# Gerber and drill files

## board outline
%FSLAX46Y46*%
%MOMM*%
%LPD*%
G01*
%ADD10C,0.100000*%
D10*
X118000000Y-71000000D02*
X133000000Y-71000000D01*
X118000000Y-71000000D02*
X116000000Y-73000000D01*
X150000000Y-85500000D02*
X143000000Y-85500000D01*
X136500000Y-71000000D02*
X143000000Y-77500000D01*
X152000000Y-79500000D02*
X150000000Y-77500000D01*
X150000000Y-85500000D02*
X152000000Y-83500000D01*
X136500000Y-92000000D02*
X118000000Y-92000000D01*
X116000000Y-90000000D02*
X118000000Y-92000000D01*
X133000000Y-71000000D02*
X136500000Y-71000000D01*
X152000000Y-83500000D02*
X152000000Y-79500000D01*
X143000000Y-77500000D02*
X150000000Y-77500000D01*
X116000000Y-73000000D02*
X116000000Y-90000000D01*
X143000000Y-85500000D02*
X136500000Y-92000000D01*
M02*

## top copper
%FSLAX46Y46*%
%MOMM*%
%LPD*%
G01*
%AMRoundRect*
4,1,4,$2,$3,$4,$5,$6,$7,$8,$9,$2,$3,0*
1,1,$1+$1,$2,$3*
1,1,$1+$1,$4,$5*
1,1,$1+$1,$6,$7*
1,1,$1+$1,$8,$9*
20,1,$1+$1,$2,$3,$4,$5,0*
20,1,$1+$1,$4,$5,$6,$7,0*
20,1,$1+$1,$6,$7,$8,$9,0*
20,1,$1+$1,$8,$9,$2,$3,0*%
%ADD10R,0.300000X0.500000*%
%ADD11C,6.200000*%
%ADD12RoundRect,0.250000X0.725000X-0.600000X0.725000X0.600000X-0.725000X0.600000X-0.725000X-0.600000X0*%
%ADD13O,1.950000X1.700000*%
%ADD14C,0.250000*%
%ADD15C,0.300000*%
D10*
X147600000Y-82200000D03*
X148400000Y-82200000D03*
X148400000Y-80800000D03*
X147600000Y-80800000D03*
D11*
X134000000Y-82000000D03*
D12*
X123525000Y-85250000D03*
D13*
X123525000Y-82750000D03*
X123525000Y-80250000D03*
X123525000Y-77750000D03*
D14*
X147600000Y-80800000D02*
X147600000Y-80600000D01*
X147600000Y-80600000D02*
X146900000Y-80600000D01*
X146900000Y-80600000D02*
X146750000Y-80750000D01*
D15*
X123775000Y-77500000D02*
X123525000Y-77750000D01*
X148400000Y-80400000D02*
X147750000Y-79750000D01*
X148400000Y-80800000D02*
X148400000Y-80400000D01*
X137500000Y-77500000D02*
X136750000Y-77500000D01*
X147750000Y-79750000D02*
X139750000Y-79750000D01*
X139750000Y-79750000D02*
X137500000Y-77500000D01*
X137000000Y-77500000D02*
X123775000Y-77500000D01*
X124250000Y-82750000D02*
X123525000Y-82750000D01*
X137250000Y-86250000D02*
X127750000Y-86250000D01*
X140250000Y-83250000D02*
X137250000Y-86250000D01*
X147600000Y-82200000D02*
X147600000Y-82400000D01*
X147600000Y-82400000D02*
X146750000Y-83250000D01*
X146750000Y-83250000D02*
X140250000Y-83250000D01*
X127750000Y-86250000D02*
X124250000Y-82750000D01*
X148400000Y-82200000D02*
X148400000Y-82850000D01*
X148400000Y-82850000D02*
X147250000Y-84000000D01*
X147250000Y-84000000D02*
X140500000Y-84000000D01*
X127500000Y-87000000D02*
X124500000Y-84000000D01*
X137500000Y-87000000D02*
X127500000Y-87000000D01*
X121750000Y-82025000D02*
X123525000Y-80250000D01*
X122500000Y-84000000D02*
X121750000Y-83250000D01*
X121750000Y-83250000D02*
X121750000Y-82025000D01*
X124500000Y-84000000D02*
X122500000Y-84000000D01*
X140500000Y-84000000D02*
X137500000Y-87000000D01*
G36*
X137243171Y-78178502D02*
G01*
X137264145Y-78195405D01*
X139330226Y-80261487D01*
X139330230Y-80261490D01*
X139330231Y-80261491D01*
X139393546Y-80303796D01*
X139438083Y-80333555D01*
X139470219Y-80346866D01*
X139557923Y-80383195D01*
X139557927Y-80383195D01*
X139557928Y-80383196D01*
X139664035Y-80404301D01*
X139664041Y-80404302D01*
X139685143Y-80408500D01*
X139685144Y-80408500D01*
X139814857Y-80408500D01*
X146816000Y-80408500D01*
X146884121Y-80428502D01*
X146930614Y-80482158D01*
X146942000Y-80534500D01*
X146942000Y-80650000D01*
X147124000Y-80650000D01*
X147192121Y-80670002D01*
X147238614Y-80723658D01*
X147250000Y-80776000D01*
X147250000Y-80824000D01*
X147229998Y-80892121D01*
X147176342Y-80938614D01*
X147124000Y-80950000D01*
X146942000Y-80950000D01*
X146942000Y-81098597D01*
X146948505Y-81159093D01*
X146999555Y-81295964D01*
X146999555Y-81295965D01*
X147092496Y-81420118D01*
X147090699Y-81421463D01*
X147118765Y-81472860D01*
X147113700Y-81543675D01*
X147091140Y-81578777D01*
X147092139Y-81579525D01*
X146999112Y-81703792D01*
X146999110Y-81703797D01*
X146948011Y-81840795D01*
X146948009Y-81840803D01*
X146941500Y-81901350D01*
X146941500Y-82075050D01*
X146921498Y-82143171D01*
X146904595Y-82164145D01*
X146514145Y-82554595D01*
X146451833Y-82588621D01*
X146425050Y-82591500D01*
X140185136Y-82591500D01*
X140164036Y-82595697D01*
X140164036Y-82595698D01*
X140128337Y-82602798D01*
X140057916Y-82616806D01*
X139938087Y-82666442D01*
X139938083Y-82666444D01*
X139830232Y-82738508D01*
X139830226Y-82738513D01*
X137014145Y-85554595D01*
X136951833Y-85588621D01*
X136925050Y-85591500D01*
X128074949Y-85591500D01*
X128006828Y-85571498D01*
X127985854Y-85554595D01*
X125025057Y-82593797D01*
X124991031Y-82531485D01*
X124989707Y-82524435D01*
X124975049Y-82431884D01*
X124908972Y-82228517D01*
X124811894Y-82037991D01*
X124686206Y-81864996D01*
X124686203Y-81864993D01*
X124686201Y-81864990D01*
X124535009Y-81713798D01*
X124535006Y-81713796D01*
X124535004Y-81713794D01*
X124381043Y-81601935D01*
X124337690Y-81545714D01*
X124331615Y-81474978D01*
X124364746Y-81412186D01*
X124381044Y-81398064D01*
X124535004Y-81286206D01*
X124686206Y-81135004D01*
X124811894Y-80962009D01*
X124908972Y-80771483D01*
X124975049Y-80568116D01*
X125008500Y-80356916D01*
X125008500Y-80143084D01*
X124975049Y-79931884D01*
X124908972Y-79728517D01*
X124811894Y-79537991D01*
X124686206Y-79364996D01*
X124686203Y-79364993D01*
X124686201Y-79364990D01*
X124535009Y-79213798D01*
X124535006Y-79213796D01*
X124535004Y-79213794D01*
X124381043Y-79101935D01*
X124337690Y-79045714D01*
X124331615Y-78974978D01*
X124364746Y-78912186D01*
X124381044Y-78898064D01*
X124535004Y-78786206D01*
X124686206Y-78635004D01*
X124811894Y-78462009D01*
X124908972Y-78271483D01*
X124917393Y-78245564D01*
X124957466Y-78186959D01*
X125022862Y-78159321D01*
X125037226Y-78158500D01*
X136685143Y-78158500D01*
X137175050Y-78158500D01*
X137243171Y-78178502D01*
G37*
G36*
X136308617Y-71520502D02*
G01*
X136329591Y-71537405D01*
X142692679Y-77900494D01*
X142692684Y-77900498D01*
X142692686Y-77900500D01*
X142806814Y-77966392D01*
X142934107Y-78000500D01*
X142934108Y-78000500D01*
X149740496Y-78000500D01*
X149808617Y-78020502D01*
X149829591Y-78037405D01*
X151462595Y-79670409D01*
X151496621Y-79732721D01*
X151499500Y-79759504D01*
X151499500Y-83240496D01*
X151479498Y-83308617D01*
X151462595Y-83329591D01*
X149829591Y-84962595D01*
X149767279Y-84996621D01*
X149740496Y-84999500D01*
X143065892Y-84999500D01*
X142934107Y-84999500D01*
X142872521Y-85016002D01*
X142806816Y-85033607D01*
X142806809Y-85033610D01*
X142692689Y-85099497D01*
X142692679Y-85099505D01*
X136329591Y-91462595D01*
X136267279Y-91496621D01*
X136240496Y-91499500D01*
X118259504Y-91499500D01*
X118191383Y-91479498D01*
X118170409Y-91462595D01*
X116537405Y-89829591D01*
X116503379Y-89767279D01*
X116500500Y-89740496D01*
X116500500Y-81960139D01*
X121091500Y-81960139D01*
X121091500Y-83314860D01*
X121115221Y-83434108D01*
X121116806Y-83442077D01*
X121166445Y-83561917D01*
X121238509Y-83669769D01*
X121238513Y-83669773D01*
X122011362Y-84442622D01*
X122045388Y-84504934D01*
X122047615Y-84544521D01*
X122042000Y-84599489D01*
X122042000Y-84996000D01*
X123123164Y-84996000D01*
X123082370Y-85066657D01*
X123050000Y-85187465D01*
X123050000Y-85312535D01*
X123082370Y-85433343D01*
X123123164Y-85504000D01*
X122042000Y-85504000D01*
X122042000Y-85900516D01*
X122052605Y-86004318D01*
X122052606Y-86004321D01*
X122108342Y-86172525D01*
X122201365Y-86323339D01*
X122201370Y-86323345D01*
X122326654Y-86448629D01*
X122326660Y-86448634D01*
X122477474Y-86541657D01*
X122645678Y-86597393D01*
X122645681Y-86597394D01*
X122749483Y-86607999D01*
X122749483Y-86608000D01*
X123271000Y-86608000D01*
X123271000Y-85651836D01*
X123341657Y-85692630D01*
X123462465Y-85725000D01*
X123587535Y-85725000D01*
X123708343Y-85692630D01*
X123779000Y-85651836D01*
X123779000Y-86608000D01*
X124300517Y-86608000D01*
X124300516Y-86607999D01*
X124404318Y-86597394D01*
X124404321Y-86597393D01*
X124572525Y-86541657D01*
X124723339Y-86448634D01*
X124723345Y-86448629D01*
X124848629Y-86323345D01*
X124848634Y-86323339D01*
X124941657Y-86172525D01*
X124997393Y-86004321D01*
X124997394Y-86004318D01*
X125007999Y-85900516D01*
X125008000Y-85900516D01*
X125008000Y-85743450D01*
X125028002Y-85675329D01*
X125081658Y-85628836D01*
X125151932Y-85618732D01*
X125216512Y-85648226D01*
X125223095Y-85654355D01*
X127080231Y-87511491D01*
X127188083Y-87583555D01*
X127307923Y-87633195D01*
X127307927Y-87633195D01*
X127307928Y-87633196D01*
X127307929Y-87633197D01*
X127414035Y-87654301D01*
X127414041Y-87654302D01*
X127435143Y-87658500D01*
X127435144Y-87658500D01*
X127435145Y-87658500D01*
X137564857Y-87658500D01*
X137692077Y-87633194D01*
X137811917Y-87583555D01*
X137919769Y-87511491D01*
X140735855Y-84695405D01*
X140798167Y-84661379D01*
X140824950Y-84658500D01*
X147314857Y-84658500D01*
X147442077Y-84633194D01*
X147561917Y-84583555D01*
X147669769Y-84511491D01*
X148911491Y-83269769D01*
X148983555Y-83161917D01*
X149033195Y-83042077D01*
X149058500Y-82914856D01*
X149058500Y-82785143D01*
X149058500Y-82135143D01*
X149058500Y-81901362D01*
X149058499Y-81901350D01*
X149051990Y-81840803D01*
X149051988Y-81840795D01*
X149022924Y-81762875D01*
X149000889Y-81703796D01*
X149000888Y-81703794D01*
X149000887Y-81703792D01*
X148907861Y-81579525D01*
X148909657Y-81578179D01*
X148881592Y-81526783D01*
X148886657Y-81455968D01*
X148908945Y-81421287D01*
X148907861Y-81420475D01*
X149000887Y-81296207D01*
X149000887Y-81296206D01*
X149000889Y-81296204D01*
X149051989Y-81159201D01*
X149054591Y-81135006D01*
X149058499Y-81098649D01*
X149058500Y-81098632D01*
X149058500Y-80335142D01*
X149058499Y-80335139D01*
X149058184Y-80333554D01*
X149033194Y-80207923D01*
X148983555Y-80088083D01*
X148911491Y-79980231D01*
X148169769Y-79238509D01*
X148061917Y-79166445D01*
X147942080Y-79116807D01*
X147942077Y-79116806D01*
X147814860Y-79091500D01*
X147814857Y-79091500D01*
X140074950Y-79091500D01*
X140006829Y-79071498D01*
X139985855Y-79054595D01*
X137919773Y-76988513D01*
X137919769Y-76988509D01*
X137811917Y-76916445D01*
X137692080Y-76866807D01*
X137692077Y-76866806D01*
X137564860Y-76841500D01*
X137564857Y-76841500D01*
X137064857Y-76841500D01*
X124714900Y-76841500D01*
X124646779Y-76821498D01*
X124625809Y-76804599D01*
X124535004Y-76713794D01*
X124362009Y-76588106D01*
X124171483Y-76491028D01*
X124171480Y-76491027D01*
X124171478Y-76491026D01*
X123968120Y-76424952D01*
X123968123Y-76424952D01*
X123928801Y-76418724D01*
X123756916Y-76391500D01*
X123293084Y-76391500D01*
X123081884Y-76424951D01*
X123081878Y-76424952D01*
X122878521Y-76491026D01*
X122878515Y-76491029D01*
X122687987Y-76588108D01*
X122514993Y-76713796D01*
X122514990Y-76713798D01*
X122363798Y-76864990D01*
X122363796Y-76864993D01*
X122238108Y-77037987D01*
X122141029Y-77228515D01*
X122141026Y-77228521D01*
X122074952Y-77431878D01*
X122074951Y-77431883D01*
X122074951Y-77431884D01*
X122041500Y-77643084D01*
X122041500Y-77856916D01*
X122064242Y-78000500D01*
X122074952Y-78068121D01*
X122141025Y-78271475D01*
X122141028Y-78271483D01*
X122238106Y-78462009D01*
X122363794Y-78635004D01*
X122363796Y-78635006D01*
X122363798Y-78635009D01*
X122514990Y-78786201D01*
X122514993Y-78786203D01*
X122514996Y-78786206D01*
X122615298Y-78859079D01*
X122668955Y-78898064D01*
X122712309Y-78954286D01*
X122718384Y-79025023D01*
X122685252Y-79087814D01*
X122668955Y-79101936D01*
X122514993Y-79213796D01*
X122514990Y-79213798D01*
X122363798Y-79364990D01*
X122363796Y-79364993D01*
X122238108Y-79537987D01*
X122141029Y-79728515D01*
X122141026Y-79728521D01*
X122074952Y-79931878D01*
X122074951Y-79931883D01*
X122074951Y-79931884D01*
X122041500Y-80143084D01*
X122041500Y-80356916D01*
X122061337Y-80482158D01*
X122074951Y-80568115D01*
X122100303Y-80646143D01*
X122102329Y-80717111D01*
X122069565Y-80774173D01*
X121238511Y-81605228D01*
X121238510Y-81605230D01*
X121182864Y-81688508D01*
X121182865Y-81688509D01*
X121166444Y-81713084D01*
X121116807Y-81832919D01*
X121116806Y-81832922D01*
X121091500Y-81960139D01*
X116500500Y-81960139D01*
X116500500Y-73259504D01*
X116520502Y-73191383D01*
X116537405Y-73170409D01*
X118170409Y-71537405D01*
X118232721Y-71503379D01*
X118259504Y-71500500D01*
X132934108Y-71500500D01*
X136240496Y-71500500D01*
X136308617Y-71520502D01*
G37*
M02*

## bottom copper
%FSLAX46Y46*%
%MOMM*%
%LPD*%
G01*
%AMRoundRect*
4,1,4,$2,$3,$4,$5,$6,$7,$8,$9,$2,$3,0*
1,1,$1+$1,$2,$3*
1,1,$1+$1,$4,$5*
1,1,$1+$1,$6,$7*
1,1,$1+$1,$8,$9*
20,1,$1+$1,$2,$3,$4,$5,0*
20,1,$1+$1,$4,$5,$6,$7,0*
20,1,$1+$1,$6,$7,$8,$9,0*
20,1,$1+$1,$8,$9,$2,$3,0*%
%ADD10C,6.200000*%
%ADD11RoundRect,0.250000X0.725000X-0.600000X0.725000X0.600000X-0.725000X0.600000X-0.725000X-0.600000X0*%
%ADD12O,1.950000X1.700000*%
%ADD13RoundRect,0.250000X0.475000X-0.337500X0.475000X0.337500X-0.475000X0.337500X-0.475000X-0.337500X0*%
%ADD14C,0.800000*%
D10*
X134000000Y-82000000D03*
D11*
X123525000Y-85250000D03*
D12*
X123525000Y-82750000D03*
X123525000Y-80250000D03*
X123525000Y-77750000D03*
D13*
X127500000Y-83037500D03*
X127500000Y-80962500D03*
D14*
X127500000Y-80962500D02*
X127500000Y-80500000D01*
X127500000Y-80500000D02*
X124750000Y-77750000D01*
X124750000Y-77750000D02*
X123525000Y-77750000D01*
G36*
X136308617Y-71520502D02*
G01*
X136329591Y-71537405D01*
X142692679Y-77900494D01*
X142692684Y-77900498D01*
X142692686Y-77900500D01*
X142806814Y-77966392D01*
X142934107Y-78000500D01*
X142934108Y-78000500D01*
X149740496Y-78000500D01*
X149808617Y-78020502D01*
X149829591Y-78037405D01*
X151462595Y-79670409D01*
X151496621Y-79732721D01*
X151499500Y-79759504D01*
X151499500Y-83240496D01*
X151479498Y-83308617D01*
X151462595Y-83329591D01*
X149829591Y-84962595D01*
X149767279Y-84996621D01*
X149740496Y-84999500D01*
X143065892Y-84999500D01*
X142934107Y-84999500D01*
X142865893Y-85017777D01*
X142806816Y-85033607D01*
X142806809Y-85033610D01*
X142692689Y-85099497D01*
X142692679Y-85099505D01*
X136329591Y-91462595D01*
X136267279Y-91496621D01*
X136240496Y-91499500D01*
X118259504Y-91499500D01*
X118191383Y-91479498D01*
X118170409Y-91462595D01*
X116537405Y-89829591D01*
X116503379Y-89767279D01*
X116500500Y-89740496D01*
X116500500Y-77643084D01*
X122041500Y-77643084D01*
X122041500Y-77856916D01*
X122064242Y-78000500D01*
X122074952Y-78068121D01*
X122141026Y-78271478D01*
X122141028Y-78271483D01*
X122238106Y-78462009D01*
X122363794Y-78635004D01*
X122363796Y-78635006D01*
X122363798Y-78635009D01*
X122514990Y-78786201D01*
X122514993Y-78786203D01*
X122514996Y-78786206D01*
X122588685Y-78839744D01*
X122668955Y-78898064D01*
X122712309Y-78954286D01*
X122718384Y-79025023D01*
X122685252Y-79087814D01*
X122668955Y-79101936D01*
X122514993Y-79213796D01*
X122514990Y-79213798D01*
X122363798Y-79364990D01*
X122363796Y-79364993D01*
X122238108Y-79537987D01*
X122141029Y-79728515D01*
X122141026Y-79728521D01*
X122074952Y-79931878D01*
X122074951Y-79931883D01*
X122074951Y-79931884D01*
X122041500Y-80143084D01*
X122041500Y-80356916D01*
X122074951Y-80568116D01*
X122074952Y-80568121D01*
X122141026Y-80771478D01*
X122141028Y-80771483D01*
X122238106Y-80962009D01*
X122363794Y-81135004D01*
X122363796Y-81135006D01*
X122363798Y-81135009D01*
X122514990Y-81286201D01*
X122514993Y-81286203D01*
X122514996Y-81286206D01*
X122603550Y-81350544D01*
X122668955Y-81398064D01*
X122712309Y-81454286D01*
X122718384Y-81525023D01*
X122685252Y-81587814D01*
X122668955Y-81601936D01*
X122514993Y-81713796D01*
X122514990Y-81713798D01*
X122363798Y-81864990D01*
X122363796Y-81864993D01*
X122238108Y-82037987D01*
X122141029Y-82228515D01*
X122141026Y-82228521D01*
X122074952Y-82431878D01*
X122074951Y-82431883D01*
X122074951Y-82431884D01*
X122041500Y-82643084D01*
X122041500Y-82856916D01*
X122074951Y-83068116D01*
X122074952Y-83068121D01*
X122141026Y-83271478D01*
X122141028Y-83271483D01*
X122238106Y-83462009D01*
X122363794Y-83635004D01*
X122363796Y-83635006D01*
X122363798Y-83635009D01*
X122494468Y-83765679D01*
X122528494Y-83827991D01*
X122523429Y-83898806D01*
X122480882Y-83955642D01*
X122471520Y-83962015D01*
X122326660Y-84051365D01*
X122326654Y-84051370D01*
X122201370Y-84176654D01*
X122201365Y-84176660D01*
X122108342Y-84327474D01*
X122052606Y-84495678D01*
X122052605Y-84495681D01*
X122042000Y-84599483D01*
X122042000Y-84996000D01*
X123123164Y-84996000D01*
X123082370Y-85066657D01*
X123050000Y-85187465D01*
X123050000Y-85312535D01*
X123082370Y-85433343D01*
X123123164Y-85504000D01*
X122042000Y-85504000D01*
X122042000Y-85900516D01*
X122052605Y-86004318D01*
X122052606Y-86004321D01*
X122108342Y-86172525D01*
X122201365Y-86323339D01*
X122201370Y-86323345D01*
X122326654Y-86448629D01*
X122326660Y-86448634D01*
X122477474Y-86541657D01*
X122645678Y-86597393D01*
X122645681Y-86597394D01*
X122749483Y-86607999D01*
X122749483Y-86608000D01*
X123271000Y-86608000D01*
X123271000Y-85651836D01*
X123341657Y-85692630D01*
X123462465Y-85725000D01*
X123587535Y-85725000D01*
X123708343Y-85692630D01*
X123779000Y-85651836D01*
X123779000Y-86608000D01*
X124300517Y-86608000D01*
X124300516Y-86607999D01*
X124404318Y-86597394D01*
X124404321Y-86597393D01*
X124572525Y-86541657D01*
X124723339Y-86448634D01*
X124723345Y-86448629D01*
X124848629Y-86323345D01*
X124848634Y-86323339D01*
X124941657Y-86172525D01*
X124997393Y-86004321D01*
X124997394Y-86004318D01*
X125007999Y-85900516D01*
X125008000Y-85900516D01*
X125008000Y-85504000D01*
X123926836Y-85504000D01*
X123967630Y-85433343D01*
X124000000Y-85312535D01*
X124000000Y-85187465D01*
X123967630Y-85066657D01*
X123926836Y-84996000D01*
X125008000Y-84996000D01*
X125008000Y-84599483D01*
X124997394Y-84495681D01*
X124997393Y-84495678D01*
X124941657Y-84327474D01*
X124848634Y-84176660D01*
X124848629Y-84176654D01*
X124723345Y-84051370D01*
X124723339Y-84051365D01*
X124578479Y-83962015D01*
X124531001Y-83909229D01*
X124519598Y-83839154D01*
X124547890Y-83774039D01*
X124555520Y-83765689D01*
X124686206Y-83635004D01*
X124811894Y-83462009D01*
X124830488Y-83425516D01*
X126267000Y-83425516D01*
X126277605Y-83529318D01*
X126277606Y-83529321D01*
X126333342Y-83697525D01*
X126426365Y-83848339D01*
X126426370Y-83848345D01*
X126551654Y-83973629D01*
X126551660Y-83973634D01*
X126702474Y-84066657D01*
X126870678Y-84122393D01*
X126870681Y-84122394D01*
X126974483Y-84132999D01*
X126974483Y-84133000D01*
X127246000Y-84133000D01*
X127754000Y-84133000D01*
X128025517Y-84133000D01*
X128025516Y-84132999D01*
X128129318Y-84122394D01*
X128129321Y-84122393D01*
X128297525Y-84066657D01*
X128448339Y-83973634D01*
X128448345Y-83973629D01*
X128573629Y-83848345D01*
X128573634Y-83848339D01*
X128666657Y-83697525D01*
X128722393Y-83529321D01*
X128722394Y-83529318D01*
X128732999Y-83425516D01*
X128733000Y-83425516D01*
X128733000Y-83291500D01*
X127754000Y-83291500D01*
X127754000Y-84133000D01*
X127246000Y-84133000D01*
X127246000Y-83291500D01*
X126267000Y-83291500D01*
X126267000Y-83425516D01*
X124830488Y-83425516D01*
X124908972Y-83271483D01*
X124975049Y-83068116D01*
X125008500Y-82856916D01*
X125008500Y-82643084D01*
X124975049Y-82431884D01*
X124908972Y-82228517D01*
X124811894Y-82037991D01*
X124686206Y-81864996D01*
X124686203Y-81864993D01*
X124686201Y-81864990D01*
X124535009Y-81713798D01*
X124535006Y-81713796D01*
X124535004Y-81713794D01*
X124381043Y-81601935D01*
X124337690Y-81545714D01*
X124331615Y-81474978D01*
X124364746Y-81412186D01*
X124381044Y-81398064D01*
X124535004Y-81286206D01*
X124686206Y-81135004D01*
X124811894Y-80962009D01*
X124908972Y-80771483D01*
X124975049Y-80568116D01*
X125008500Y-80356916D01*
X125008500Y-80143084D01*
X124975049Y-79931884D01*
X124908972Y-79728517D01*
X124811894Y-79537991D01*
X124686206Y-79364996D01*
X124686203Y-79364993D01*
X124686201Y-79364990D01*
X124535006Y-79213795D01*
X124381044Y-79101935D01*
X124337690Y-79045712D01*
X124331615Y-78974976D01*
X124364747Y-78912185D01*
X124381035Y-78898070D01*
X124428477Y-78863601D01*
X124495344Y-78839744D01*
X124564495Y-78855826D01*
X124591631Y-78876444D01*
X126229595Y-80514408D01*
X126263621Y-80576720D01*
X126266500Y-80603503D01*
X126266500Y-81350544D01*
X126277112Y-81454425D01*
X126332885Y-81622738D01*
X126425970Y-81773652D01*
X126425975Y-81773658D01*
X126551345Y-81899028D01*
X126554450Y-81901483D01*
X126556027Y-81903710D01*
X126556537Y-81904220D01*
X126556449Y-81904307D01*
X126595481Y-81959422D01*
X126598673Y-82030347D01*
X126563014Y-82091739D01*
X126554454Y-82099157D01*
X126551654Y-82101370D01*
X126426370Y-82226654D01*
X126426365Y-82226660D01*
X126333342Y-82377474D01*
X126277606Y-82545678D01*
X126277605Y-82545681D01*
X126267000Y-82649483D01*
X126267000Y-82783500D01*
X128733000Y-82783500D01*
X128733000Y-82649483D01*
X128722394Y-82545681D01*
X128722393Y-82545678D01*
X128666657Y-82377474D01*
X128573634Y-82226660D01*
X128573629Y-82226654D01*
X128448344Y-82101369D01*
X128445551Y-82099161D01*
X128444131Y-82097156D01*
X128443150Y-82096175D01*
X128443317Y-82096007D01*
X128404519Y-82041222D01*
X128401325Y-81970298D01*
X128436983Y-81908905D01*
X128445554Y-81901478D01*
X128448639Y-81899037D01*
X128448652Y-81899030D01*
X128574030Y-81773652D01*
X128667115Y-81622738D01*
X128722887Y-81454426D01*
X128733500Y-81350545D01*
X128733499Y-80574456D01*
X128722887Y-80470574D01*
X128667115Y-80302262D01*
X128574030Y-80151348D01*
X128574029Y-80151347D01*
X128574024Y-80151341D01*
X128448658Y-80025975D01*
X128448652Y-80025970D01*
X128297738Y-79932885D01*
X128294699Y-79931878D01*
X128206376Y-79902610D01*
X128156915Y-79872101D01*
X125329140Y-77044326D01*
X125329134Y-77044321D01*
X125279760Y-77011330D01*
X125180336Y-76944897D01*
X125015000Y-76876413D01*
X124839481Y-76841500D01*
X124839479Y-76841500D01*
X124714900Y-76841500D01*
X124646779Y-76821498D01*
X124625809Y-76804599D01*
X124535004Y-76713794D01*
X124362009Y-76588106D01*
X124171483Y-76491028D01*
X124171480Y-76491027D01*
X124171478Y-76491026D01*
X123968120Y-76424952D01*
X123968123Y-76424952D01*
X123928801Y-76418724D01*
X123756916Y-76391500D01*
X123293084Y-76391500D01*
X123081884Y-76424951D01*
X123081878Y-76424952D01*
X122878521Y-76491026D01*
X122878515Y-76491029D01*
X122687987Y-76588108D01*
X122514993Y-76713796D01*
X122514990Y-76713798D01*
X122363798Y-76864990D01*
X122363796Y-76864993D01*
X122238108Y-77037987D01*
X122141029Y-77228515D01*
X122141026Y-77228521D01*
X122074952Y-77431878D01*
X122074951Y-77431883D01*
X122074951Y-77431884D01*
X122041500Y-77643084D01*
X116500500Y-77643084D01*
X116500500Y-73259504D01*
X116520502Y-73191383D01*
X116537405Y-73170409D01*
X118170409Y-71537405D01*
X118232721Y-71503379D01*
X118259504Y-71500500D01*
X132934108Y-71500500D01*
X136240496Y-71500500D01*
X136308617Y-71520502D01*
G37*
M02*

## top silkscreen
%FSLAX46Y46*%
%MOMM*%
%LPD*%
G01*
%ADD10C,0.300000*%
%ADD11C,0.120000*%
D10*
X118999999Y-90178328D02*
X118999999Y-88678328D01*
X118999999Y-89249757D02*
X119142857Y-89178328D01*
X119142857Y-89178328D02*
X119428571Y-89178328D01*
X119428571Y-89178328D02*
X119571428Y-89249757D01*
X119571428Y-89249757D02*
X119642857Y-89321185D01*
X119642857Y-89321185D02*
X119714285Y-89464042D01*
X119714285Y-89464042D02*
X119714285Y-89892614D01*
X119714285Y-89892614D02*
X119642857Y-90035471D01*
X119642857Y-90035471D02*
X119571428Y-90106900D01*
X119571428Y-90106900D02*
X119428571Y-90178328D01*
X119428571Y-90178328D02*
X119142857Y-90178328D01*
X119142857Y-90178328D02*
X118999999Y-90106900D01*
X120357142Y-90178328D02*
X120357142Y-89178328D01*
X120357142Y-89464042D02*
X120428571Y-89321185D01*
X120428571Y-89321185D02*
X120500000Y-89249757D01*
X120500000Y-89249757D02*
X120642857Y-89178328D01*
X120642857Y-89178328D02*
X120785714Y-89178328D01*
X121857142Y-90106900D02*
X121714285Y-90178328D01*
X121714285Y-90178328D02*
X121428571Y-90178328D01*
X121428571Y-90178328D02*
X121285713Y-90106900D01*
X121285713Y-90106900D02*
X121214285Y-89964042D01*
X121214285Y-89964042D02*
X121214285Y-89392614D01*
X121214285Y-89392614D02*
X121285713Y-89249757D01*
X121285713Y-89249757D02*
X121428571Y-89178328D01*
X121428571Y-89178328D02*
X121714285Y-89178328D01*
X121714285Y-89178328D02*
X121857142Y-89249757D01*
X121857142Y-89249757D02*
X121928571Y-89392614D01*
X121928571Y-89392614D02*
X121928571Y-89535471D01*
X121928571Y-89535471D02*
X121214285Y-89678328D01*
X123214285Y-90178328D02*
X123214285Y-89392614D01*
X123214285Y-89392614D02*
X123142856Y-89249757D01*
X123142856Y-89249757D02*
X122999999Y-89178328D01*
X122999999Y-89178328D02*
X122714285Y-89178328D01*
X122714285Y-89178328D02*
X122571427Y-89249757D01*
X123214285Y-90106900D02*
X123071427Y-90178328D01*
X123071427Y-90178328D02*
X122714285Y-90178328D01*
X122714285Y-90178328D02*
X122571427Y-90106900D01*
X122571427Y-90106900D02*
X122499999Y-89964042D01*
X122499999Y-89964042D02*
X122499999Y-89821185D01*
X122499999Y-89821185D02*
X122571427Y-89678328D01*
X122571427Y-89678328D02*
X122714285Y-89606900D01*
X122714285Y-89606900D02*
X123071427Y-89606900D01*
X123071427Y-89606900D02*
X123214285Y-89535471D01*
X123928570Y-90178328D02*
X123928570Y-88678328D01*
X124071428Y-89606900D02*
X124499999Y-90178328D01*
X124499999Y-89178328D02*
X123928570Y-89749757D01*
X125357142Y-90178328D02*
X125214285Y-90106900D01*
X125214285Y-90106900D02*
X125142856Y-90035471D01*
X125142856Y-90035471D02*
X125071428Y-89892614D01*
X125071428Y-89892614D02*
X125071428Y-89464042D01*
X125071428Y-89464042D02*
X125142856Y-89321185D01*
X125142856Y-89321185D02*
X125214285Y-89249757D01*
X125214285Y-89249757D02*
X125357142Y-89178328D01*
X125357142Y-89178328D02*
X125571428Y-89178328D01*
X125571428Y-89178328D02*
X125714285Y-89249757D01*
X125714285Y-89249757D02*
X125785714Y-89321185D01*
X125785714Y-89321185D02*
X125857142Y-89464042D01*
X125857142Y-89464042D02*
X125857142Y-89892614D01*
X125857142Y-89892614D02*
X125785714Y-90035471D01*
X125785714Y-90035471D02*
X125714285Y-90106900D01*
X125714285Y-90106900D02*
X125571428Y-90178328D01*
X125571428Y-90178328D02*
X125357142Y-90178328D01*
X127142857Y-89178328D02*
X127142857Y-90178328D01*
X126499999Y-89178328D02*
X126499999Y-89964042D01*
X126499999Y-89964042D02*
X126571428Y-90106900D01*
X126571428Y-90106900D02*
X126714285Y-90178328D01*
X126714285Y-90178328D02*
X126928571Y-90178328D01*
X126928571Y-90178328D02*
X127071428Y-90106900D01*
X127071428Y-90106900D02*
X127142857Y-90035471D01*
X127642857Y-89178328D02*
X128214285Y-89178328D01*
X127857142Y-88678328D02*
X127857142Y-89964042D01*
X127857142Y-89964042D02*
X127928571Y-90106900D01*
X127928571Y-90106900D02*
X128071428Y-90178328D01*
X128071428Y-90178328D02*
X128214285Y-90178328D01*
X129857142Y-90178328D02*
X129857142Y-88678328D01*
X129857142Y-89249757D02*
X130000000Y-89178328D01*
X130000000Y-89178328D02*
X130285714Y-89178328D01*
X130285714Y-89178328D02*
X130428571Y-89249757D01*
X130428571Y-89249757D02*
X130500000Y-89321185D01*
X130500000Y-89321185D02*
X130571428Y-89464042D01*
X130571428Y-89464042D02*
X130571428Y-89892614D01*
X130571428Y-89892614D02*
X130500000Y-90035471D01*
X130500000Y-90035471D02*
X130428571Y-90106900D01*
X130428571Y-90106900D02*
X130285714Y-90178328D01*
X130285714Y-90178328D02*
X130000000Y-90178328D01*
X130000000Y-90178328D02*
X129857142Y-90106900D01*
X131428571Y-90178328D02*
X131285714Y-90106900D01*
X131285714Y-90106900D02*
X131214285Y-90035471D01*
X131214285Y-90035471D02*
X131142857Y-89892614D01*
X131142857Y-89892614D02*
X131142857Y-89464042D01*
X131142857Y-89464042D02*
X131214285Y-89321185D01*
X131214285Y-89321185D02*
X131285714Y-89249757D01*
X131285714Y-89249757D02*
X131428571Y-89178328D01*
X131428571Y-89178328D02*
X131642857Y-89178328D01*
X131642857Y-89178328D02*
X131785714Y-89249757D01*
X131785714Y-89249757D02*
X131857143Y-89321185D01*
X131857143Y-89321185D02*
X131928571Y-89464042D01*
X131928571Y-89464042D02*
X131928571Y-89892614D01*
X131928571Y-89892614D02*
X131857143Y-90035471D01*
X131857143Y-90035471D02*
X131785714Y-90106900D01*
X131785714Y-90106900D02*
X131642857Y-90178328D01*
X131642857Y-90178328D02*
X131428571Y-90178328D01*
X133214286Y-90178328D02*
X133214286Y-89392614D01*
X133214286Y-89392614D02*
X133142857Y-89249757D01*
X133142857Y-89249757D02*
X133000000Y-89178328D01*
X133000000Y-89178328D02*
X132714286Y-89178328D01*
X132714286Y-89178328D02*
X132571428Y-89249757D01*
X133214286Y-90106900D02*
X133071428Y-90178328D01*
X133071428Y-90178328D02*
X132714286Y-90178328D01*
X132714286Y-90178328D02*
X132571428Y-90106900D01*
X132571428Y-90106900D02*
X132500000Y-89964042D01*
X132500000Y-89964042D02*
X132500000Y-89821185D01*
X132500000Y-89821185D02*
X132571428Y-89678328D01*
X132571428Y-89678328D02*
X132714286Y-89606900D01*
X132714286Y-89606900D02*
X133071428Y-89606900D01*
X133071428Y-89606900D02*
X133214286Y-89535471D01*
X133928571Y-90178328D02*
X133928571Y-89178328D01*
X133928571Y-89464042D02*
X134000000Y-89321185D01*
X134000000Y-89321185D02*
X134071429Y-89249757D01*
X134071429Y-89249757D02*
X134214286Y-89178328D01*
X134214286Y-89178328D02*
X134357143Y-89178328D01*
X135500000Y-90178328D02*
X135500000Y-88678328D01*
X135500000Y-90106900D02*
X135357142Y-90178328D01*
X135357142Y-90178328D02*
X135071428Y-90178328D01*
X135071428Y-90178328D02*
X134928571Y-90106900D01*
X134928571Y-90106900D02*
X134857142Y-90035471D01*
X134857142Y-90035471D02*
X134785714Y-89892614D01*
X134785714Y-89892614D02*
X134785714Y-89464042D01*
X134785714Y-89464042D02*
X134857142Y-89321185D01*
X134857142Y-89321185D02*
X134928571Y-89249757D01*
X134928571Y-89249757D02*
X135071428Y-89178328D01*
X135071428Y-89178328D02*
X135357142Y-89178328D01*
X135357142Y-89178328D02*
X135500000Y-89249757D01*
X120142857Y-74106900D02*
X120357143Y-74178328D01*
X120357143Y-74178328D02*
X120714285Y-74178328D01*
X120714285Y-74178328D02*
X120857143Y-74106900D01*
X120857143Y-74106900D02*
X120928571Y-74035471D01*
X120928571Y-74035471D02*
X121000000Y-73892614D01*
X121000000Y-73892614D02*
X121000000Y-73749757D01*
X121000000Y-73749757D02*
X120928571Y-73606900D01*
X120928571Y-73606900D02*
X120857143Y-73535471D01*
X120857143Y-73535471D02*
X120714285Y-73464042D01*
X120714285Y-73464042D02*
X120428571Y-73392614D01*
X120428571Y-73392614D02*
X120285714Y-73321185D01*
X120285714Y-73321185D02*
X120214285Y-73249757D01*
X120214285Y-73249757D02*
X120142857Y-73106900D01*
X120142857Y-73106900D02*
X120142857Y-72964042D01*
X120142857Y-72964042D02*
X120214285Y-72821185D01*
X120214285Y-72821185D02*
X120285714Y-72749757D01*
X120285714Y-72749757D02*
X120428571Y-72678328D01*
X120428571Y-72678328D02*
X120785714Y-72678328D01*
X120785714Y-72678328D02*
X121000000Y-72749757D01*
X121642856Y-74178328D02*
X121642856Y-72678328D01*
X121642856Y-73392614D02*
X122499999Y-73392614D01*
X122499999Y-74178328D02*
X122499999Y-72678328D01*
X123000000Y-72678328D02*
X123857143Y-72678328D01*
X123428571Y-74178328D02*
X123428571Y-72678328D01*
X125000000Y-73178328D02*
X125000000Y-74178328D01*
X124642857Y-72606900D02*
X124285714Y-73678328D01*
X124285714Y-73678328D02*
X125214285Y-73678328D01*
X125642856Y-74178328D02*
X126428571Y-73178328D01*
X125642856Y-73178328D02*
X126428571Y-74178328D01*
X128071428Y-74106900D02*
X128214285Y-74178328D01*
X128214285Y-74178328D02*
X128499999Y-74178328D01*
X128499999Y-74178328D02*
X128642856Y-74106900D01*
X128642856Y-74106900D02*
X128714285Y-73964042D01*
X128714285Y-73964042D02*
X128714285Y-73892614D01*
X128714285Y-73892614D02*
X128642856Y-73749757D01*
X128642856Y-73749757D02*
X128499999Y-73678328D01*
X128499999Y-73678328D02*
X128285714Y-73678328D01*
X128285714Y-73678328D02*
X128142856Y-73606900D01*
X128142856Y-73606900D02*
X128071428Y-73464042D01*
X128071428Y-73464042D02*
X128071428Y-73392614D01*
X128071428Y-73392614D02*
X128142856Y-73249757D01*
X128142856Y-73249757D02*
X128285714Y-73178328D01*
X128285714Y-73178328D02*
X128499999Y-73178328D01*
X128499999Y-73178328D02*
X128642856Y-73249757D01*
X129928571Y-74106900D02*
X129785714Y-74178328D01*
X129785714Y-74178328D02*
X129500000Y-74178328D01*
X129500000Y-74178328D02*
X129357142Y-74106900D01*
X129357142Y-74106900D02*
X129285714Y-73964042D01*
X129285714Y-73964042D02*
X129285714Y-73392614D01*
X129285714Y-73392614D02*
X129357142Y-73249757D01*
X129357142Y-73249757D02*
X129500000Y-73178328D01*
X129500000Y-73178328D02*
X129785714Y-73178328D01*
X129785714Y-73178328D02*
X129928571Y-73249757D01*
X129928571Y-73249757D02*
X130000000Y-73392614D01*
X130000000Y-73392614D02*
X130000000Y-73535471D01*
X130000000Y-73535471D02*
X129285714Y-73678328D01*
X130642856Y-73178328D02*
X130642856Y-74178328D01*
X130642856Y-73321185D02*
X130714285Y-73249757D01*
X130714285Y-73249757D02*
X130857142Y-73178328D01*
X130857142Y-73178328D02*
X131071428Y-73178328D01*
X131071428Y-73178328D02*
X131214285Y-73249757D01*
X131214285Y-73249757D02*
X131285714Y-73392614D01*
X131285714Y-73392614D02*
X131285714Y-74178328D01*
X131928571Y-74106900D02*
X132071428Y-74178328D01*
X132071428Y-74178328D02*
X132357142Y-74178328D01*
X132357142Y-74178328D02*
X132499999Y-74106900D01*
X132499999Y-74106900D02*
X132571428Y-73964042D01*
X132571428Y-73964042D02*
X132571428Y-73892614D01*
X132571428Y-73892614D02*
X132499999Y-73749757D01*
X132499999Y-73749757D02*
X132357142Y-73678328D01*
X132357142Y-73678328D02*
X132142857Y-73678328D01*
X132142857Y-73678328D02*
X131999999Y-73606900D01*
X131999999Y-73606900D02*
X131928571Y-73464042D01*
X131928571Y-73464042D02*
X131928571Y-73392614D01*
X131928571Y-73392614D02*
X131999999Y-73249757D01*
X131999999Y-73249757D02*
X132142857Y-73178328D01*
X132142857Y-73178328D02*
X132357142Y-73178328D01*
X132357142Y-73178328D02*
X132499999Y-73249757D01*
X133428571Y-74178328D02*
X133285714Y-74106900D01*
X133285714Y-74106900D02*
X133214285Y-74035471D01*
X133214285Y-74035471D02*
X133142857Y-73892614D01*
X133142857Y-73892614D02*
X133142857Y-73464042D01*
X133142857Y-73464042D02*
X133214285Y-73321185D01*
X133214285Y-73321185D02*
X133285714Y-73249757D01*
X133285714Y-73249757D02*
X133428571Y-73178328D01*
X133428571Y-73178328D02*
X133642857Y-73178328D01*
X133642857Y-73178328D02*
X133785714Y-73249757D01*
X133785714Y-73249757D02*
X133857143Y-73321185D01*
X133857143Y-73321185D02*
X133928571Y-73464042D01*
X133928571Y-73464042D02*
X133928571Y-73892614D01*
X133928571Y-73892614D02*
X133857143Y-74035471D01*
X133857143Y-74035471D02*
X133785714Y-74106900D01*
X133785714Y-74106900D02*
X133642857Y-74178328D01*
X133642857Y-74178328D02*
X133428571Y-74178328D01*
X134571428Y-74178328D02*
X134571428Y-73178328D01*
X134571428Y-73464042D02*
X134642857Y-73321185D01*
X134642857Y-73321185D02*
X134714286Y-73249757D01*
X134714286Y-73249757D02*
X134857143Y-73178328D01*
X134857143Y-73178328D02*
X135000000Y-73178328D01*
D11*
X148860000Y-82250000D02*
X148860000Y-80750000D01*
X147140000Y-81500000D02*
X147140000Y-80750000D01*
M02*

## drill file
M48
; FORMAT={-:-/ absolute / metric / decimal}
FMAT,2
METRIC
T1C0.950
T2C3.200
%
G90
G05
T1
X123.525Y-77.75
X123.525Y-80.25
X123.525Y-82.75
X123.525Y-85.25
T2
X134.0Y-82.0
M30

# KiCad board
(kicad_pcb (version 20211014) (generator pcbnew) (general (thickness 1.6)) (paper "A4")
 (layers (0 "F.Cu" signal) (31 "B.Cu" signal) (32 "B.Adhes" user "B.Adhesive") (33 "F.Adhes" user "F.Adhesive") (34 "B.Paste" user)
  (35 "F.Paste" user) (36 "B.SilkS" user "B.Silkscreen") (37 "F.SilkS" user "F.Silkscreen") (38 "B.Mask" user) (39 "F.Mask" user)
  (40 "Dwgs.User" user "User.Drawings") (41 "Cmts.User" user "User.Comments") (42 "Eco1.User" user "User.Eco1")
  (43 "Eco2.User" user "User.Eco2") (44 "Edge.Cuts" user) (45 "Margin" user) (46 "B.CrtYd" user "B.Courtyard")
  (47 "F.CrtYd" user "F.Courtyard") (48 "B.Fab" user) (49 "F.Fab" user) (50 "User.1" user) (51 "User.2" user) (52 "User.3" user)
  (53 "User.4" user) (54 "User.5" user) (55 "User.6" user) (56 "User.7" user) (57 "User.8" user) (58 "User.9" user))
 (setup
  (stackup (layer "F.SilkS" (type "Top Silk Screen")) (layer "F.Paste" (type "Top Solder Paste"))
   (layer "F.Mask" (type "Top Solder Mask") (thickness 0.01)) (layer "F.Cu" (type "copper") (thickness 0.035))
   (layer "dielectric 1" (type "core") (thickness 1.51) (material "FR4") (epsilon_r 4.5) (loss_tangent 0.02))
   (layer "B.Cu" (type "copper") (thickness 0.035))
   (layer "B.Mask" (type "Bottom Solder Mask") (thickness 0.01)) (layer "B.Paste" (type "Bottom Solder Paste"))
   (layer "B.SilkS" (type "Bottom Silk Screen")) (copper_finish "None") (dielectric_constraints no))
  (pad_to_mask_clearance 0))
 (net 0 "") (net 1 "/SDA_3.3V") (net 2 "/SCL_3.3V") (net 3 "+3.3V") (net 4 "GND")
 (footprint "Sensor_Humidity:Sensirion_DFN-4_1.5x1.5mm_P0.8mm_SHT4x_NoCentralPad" (layer "F.Cu") (at 148 81.5 90)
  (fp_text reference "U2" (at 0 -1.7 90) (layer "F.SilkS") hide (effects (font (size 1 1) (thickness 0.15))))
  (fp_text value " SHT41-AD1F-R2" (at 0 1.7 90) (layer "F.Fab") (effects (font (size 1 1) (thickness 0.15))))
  (fp_line (start -0.75 0.86) (end 0.75 0.86) (layer "F.SilkS") (width 0.12))
  (fp_line (start 0 -0.86) (end 0.75 -0.86) (layer "F.SilkS") (width 0.12))
  (pad "1" smd rect (at -0.7 -0.4 90) (size 0.5 0.3) (layers "F.Cu" "F.Paste" "F.Mask") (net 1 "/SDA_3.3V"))
  (pad "2" smd rect (at -0.7 0.4 90) (size 0.5 0.3) (layers "F.Cu" "F.Paste" "F.Mask") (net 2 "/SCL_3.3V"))
  (pad "3" smd rect (at 0.7 0.4 90) (size 0.5 0.3) (layers "F.Cu" "F.Paste" "F.Mask") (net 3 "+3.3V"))
  (pad "4" smd rect (at 0.7 -0.4 90) (size 0.5 0.3) (layers "F.Cu" "F.Paste" "F.Mask") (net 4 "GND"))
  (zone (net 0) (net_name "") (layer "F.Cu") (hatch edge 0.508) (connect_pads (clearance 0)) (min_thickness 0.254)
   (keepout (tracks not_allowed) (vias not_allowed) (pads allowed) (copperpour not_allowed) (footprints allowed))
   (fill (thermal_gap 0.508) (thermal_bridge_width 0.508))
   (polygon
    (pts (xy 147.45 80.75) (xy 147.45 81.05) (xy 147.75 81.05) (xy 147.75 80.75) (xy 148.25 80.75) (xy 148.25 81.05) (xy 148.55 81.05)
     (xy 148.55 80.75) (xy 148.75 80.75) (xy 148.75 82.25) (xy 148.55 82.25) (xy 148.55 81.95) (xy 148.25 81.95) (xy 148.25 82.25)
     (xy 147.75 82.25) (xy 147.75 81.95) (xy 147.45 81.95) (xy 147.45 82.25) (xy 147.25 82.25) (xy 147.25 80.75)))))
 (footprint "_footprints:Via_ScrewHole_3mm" (layer "F.Cu") (at 134 82)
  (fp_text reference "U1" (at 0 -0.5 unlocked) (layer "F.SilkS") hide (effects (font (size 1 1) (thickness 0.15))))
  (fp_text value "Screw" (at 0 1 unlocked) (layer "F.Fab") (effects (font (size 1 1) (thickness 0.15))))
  (pad "1" thru_hole circle (at 0 0) (size 6.2 6.2) (drill 3.2) (layers *.Cu *.Mask) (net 4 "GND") (zone_connect 2)))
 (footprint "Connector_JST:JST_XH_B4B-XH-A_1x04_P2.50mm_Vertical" (layer "B.Cu") (at 123.525 85.25 90)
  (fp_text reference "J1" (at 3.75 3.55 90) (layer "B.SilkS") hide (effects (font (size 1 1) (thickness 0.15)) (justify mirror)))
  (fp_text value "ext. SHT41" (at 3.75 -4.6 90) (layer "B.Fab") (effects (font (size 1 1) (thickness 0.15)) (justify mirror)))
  (pad "1" thru_hole roundrect (at 0 0 90) (size 1.7 1.95) (drill 0.95) (layers *.Cu *.Mask) (roundrect_rratio 0.1470588235) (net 4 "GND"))
  (pad "2" thru_hole oval (at 2.5 0 90) (size 1.7 1.95) (drill 0.95) (layers *.Cu *.Mask) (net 1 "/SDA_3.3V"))
  (pad "3" thru_hole oval (at 5 0 90) (size 1.7 1.95) (drill 0.95) (layers *.Cu *.Mask) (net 2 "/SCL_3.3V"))
  (pad "4" thru_hole oval (at 7.5 0 90) (size 1.7 1.95) (drill 0.95) (layers *.Cu *.Mask) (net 3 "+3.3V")))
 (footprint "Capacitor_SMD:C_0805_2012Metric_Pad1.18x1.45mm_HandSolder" (layer "B.Cu") (at 127.5 82 90)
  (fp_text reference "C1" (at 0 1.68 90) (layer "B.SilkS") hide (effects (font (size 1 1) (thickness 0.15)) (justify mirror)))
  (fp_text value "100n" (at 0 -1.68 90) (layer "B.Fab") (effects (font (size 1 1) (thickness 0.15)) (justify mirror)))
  (pad "1" smd roundrect (at -1.0375 0 90) (size 1.175 1.45) (layers "B.Cu" "B.Paste" "B.Mask") (roundrect_rratio 0.2127659574)
   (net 4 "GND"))
  (pad "2" smd roundrect (at 1.0375 0 90) (size 1.175 1.45) (layers "B.Cu" "B.Paste" "B.Mask") (roundrect_rratio 0.2127659574)
   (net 3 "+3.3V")))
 (gr_line (start 118 71) (end 133 71) (layer "Edge.Cuts") (width 0.1))
 (gr_line (start 118 71) (end 116 73) (layer "Edge.Cuts") (width 0.1))
 (gr_line (start 150 85.5) (end 143 85.5) (layer "Edge.Cuts") (width 0.1))
 (gr_line (start 136.5 71) (end 143 77.5) (layer "Edge.Cuts") (width 0.1))
 (gr_line (start 152 79.5) (end 150 77.5) (layer "Edge.Cuts") (width 0.1))
 (gr_line (start 150 85.5) (end 152 83.5) (layer "Edge.Cuts") (width 0.1))
 (gr_line (start 136.5 92) (end 118 92) (layer "Edge.Cuts") (width 0.1))
 (gr_line (start 116 90) (end 118 92) (layer "Edge.Cuts") (width 0.1))
 (gr_line (start 133 71) (end 136.5 71) (layer "Edge.Cuts") (width 0.1))
 (gr_line (start 152 83.5) (end 152 79.5) (layer "Edge.Cuts") (width 0.1))
 (gr_line (start 143 77.5) (end 150 77.5) (layer "Edge.Cuts") (width 0.1))
 (gr_line (start 116 73) (end 116 90) (layer "Edge.Cuts") (width 0.1))
 (gr_line (start 143 85.5) (end 136.5 92) (layer "Edge.Cuts") (width 0.1))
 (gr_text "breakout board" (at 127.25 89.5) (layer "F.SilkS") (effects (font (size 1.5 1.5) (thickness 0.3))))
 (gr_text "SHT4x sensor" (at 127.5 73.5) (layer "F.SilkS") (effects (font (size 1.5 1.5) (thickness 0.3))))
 (segment (start 147.6 80.8) (end 147.6 80.6) (width 0.25) (layer "F.Cu") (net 4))
 (segment (start 147.6 80.6) (end 146.9 80.6) (width 0.25) (layer "F.Cu") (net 4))
 (segment (start 146.9 80.6) (end 146.75 80.75) (width 0.25) (layer "F.Cu") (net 4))
 (segment (start 123.775 77.5) (end 123.525 77.75) (width 0.3) (layer "F.Cu") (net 3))
 (segment (start 148.4 80.4) (end 147.75 79.75) (width 0.3) (layer "F.Cu") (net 3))
 (segment (start 148.4 80.8) (end 148.4 80.4) (width 0.3) (layer "F.Cu") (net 3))
 (segment (start 137.5 77.5) (end 136.75 77.5) (width 0.3) (layer "F.Cu") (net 3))
 (segment (start 147.75 79.75) (end 139.75 79.75) (width 0.3) (layer "F.Cu") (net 3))
 (segment (start 139.75 79.75) (end 137.5 77.5) (width 0.3) (layer "F.Cu") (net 3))
 (segment (start 137 77.5) (end 123.775 77.5) (width 0.3) (layer "F.Cu") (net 3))
 (segment (start 127.5 80.9625) (end 127.5 80.5) (width 0.8) (layer "B.Cu") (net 3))
 (segment (start 127.5 80.5) (end 124.75 77.75) (width 0.8) (layer "B.Cu") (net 3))
 (segment (start 124.75 77.75) (end 123.525 77.75) (width 0.8) (layer "B.Cu") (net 3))
 (segment (start 124.25 82.75) (end 123.525 82.75) (width 0.3) (layer "F.Cu") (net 1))
 (segment (start 137.25 86.25) (end 127.75 86.25) (width 0.3) (layer "F.Cu") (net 1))
 (segment (start 140.25 83.25) (end 137.25 86.25) (width 0.3) (layer "F.Cu") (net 1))
 (segment (start 147.6 82.2) (end 147.6 82.4) (width 0.3) (layer "F.Cu") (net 1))
 (segment (start 147.6 82.4) (end 146.75 83.25) (width 0.3) (layer "F.Cu") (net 1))
 (segment (start 146.75 83.25) (end 140.25 83.25) (width 0.3) (layer "F.Cu") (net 1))
 (segment (start 127.75 86.25) (end 124.25 82.75) (width 0.3) (layer "F.Cu") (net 1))
 (segment (start 148.4 82.2) (end 148.4 82.85) (width 0.3) (layer "F.Cu") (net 2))
 (segment (start 148.4 82.85) (end 147.25 84) (width 0.3) (layer "F.Cu") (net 2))
 (segment (start 147.25 84) (end 140.5 84) (width 0.3) (layer "F.Cu") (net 2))
 (segment (start 127.5 87) (end 124.5 84) (width 0.3) (layer "F.Cu") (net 2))
 (segment (start 137.5 87) (end 127.5 87) (width 0.3) (layer "F.Cu") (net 2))
 (segment (start 121.75 82.025) (end 123.525 80.25) (width 0.3) (layer "F.Cu") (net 2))
 (segment (start 122.5 84) (end 121.75 83.25) (width 0.3) (layer "F.Cu") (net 2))
 (segment (start 121.75 83.25) (end 121.75 82.025) (width 0.3) (layer "F.Cu") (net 2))
 (segment (start 124.5 84) (end 122.5 84) (width 0.3) (layer "F.Cu") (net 2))
 (segment (start 140.5 84) (end 137.5 87) (width 0.3) (layer "F.Cu") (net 2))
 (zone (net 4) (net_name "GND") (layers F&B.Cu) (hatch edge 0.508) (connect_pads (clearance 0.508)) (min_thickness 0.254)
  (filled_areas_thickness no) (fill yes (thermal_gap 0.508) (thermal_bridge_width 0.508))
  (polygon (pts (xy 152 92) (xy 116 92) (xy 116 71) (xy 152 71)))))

